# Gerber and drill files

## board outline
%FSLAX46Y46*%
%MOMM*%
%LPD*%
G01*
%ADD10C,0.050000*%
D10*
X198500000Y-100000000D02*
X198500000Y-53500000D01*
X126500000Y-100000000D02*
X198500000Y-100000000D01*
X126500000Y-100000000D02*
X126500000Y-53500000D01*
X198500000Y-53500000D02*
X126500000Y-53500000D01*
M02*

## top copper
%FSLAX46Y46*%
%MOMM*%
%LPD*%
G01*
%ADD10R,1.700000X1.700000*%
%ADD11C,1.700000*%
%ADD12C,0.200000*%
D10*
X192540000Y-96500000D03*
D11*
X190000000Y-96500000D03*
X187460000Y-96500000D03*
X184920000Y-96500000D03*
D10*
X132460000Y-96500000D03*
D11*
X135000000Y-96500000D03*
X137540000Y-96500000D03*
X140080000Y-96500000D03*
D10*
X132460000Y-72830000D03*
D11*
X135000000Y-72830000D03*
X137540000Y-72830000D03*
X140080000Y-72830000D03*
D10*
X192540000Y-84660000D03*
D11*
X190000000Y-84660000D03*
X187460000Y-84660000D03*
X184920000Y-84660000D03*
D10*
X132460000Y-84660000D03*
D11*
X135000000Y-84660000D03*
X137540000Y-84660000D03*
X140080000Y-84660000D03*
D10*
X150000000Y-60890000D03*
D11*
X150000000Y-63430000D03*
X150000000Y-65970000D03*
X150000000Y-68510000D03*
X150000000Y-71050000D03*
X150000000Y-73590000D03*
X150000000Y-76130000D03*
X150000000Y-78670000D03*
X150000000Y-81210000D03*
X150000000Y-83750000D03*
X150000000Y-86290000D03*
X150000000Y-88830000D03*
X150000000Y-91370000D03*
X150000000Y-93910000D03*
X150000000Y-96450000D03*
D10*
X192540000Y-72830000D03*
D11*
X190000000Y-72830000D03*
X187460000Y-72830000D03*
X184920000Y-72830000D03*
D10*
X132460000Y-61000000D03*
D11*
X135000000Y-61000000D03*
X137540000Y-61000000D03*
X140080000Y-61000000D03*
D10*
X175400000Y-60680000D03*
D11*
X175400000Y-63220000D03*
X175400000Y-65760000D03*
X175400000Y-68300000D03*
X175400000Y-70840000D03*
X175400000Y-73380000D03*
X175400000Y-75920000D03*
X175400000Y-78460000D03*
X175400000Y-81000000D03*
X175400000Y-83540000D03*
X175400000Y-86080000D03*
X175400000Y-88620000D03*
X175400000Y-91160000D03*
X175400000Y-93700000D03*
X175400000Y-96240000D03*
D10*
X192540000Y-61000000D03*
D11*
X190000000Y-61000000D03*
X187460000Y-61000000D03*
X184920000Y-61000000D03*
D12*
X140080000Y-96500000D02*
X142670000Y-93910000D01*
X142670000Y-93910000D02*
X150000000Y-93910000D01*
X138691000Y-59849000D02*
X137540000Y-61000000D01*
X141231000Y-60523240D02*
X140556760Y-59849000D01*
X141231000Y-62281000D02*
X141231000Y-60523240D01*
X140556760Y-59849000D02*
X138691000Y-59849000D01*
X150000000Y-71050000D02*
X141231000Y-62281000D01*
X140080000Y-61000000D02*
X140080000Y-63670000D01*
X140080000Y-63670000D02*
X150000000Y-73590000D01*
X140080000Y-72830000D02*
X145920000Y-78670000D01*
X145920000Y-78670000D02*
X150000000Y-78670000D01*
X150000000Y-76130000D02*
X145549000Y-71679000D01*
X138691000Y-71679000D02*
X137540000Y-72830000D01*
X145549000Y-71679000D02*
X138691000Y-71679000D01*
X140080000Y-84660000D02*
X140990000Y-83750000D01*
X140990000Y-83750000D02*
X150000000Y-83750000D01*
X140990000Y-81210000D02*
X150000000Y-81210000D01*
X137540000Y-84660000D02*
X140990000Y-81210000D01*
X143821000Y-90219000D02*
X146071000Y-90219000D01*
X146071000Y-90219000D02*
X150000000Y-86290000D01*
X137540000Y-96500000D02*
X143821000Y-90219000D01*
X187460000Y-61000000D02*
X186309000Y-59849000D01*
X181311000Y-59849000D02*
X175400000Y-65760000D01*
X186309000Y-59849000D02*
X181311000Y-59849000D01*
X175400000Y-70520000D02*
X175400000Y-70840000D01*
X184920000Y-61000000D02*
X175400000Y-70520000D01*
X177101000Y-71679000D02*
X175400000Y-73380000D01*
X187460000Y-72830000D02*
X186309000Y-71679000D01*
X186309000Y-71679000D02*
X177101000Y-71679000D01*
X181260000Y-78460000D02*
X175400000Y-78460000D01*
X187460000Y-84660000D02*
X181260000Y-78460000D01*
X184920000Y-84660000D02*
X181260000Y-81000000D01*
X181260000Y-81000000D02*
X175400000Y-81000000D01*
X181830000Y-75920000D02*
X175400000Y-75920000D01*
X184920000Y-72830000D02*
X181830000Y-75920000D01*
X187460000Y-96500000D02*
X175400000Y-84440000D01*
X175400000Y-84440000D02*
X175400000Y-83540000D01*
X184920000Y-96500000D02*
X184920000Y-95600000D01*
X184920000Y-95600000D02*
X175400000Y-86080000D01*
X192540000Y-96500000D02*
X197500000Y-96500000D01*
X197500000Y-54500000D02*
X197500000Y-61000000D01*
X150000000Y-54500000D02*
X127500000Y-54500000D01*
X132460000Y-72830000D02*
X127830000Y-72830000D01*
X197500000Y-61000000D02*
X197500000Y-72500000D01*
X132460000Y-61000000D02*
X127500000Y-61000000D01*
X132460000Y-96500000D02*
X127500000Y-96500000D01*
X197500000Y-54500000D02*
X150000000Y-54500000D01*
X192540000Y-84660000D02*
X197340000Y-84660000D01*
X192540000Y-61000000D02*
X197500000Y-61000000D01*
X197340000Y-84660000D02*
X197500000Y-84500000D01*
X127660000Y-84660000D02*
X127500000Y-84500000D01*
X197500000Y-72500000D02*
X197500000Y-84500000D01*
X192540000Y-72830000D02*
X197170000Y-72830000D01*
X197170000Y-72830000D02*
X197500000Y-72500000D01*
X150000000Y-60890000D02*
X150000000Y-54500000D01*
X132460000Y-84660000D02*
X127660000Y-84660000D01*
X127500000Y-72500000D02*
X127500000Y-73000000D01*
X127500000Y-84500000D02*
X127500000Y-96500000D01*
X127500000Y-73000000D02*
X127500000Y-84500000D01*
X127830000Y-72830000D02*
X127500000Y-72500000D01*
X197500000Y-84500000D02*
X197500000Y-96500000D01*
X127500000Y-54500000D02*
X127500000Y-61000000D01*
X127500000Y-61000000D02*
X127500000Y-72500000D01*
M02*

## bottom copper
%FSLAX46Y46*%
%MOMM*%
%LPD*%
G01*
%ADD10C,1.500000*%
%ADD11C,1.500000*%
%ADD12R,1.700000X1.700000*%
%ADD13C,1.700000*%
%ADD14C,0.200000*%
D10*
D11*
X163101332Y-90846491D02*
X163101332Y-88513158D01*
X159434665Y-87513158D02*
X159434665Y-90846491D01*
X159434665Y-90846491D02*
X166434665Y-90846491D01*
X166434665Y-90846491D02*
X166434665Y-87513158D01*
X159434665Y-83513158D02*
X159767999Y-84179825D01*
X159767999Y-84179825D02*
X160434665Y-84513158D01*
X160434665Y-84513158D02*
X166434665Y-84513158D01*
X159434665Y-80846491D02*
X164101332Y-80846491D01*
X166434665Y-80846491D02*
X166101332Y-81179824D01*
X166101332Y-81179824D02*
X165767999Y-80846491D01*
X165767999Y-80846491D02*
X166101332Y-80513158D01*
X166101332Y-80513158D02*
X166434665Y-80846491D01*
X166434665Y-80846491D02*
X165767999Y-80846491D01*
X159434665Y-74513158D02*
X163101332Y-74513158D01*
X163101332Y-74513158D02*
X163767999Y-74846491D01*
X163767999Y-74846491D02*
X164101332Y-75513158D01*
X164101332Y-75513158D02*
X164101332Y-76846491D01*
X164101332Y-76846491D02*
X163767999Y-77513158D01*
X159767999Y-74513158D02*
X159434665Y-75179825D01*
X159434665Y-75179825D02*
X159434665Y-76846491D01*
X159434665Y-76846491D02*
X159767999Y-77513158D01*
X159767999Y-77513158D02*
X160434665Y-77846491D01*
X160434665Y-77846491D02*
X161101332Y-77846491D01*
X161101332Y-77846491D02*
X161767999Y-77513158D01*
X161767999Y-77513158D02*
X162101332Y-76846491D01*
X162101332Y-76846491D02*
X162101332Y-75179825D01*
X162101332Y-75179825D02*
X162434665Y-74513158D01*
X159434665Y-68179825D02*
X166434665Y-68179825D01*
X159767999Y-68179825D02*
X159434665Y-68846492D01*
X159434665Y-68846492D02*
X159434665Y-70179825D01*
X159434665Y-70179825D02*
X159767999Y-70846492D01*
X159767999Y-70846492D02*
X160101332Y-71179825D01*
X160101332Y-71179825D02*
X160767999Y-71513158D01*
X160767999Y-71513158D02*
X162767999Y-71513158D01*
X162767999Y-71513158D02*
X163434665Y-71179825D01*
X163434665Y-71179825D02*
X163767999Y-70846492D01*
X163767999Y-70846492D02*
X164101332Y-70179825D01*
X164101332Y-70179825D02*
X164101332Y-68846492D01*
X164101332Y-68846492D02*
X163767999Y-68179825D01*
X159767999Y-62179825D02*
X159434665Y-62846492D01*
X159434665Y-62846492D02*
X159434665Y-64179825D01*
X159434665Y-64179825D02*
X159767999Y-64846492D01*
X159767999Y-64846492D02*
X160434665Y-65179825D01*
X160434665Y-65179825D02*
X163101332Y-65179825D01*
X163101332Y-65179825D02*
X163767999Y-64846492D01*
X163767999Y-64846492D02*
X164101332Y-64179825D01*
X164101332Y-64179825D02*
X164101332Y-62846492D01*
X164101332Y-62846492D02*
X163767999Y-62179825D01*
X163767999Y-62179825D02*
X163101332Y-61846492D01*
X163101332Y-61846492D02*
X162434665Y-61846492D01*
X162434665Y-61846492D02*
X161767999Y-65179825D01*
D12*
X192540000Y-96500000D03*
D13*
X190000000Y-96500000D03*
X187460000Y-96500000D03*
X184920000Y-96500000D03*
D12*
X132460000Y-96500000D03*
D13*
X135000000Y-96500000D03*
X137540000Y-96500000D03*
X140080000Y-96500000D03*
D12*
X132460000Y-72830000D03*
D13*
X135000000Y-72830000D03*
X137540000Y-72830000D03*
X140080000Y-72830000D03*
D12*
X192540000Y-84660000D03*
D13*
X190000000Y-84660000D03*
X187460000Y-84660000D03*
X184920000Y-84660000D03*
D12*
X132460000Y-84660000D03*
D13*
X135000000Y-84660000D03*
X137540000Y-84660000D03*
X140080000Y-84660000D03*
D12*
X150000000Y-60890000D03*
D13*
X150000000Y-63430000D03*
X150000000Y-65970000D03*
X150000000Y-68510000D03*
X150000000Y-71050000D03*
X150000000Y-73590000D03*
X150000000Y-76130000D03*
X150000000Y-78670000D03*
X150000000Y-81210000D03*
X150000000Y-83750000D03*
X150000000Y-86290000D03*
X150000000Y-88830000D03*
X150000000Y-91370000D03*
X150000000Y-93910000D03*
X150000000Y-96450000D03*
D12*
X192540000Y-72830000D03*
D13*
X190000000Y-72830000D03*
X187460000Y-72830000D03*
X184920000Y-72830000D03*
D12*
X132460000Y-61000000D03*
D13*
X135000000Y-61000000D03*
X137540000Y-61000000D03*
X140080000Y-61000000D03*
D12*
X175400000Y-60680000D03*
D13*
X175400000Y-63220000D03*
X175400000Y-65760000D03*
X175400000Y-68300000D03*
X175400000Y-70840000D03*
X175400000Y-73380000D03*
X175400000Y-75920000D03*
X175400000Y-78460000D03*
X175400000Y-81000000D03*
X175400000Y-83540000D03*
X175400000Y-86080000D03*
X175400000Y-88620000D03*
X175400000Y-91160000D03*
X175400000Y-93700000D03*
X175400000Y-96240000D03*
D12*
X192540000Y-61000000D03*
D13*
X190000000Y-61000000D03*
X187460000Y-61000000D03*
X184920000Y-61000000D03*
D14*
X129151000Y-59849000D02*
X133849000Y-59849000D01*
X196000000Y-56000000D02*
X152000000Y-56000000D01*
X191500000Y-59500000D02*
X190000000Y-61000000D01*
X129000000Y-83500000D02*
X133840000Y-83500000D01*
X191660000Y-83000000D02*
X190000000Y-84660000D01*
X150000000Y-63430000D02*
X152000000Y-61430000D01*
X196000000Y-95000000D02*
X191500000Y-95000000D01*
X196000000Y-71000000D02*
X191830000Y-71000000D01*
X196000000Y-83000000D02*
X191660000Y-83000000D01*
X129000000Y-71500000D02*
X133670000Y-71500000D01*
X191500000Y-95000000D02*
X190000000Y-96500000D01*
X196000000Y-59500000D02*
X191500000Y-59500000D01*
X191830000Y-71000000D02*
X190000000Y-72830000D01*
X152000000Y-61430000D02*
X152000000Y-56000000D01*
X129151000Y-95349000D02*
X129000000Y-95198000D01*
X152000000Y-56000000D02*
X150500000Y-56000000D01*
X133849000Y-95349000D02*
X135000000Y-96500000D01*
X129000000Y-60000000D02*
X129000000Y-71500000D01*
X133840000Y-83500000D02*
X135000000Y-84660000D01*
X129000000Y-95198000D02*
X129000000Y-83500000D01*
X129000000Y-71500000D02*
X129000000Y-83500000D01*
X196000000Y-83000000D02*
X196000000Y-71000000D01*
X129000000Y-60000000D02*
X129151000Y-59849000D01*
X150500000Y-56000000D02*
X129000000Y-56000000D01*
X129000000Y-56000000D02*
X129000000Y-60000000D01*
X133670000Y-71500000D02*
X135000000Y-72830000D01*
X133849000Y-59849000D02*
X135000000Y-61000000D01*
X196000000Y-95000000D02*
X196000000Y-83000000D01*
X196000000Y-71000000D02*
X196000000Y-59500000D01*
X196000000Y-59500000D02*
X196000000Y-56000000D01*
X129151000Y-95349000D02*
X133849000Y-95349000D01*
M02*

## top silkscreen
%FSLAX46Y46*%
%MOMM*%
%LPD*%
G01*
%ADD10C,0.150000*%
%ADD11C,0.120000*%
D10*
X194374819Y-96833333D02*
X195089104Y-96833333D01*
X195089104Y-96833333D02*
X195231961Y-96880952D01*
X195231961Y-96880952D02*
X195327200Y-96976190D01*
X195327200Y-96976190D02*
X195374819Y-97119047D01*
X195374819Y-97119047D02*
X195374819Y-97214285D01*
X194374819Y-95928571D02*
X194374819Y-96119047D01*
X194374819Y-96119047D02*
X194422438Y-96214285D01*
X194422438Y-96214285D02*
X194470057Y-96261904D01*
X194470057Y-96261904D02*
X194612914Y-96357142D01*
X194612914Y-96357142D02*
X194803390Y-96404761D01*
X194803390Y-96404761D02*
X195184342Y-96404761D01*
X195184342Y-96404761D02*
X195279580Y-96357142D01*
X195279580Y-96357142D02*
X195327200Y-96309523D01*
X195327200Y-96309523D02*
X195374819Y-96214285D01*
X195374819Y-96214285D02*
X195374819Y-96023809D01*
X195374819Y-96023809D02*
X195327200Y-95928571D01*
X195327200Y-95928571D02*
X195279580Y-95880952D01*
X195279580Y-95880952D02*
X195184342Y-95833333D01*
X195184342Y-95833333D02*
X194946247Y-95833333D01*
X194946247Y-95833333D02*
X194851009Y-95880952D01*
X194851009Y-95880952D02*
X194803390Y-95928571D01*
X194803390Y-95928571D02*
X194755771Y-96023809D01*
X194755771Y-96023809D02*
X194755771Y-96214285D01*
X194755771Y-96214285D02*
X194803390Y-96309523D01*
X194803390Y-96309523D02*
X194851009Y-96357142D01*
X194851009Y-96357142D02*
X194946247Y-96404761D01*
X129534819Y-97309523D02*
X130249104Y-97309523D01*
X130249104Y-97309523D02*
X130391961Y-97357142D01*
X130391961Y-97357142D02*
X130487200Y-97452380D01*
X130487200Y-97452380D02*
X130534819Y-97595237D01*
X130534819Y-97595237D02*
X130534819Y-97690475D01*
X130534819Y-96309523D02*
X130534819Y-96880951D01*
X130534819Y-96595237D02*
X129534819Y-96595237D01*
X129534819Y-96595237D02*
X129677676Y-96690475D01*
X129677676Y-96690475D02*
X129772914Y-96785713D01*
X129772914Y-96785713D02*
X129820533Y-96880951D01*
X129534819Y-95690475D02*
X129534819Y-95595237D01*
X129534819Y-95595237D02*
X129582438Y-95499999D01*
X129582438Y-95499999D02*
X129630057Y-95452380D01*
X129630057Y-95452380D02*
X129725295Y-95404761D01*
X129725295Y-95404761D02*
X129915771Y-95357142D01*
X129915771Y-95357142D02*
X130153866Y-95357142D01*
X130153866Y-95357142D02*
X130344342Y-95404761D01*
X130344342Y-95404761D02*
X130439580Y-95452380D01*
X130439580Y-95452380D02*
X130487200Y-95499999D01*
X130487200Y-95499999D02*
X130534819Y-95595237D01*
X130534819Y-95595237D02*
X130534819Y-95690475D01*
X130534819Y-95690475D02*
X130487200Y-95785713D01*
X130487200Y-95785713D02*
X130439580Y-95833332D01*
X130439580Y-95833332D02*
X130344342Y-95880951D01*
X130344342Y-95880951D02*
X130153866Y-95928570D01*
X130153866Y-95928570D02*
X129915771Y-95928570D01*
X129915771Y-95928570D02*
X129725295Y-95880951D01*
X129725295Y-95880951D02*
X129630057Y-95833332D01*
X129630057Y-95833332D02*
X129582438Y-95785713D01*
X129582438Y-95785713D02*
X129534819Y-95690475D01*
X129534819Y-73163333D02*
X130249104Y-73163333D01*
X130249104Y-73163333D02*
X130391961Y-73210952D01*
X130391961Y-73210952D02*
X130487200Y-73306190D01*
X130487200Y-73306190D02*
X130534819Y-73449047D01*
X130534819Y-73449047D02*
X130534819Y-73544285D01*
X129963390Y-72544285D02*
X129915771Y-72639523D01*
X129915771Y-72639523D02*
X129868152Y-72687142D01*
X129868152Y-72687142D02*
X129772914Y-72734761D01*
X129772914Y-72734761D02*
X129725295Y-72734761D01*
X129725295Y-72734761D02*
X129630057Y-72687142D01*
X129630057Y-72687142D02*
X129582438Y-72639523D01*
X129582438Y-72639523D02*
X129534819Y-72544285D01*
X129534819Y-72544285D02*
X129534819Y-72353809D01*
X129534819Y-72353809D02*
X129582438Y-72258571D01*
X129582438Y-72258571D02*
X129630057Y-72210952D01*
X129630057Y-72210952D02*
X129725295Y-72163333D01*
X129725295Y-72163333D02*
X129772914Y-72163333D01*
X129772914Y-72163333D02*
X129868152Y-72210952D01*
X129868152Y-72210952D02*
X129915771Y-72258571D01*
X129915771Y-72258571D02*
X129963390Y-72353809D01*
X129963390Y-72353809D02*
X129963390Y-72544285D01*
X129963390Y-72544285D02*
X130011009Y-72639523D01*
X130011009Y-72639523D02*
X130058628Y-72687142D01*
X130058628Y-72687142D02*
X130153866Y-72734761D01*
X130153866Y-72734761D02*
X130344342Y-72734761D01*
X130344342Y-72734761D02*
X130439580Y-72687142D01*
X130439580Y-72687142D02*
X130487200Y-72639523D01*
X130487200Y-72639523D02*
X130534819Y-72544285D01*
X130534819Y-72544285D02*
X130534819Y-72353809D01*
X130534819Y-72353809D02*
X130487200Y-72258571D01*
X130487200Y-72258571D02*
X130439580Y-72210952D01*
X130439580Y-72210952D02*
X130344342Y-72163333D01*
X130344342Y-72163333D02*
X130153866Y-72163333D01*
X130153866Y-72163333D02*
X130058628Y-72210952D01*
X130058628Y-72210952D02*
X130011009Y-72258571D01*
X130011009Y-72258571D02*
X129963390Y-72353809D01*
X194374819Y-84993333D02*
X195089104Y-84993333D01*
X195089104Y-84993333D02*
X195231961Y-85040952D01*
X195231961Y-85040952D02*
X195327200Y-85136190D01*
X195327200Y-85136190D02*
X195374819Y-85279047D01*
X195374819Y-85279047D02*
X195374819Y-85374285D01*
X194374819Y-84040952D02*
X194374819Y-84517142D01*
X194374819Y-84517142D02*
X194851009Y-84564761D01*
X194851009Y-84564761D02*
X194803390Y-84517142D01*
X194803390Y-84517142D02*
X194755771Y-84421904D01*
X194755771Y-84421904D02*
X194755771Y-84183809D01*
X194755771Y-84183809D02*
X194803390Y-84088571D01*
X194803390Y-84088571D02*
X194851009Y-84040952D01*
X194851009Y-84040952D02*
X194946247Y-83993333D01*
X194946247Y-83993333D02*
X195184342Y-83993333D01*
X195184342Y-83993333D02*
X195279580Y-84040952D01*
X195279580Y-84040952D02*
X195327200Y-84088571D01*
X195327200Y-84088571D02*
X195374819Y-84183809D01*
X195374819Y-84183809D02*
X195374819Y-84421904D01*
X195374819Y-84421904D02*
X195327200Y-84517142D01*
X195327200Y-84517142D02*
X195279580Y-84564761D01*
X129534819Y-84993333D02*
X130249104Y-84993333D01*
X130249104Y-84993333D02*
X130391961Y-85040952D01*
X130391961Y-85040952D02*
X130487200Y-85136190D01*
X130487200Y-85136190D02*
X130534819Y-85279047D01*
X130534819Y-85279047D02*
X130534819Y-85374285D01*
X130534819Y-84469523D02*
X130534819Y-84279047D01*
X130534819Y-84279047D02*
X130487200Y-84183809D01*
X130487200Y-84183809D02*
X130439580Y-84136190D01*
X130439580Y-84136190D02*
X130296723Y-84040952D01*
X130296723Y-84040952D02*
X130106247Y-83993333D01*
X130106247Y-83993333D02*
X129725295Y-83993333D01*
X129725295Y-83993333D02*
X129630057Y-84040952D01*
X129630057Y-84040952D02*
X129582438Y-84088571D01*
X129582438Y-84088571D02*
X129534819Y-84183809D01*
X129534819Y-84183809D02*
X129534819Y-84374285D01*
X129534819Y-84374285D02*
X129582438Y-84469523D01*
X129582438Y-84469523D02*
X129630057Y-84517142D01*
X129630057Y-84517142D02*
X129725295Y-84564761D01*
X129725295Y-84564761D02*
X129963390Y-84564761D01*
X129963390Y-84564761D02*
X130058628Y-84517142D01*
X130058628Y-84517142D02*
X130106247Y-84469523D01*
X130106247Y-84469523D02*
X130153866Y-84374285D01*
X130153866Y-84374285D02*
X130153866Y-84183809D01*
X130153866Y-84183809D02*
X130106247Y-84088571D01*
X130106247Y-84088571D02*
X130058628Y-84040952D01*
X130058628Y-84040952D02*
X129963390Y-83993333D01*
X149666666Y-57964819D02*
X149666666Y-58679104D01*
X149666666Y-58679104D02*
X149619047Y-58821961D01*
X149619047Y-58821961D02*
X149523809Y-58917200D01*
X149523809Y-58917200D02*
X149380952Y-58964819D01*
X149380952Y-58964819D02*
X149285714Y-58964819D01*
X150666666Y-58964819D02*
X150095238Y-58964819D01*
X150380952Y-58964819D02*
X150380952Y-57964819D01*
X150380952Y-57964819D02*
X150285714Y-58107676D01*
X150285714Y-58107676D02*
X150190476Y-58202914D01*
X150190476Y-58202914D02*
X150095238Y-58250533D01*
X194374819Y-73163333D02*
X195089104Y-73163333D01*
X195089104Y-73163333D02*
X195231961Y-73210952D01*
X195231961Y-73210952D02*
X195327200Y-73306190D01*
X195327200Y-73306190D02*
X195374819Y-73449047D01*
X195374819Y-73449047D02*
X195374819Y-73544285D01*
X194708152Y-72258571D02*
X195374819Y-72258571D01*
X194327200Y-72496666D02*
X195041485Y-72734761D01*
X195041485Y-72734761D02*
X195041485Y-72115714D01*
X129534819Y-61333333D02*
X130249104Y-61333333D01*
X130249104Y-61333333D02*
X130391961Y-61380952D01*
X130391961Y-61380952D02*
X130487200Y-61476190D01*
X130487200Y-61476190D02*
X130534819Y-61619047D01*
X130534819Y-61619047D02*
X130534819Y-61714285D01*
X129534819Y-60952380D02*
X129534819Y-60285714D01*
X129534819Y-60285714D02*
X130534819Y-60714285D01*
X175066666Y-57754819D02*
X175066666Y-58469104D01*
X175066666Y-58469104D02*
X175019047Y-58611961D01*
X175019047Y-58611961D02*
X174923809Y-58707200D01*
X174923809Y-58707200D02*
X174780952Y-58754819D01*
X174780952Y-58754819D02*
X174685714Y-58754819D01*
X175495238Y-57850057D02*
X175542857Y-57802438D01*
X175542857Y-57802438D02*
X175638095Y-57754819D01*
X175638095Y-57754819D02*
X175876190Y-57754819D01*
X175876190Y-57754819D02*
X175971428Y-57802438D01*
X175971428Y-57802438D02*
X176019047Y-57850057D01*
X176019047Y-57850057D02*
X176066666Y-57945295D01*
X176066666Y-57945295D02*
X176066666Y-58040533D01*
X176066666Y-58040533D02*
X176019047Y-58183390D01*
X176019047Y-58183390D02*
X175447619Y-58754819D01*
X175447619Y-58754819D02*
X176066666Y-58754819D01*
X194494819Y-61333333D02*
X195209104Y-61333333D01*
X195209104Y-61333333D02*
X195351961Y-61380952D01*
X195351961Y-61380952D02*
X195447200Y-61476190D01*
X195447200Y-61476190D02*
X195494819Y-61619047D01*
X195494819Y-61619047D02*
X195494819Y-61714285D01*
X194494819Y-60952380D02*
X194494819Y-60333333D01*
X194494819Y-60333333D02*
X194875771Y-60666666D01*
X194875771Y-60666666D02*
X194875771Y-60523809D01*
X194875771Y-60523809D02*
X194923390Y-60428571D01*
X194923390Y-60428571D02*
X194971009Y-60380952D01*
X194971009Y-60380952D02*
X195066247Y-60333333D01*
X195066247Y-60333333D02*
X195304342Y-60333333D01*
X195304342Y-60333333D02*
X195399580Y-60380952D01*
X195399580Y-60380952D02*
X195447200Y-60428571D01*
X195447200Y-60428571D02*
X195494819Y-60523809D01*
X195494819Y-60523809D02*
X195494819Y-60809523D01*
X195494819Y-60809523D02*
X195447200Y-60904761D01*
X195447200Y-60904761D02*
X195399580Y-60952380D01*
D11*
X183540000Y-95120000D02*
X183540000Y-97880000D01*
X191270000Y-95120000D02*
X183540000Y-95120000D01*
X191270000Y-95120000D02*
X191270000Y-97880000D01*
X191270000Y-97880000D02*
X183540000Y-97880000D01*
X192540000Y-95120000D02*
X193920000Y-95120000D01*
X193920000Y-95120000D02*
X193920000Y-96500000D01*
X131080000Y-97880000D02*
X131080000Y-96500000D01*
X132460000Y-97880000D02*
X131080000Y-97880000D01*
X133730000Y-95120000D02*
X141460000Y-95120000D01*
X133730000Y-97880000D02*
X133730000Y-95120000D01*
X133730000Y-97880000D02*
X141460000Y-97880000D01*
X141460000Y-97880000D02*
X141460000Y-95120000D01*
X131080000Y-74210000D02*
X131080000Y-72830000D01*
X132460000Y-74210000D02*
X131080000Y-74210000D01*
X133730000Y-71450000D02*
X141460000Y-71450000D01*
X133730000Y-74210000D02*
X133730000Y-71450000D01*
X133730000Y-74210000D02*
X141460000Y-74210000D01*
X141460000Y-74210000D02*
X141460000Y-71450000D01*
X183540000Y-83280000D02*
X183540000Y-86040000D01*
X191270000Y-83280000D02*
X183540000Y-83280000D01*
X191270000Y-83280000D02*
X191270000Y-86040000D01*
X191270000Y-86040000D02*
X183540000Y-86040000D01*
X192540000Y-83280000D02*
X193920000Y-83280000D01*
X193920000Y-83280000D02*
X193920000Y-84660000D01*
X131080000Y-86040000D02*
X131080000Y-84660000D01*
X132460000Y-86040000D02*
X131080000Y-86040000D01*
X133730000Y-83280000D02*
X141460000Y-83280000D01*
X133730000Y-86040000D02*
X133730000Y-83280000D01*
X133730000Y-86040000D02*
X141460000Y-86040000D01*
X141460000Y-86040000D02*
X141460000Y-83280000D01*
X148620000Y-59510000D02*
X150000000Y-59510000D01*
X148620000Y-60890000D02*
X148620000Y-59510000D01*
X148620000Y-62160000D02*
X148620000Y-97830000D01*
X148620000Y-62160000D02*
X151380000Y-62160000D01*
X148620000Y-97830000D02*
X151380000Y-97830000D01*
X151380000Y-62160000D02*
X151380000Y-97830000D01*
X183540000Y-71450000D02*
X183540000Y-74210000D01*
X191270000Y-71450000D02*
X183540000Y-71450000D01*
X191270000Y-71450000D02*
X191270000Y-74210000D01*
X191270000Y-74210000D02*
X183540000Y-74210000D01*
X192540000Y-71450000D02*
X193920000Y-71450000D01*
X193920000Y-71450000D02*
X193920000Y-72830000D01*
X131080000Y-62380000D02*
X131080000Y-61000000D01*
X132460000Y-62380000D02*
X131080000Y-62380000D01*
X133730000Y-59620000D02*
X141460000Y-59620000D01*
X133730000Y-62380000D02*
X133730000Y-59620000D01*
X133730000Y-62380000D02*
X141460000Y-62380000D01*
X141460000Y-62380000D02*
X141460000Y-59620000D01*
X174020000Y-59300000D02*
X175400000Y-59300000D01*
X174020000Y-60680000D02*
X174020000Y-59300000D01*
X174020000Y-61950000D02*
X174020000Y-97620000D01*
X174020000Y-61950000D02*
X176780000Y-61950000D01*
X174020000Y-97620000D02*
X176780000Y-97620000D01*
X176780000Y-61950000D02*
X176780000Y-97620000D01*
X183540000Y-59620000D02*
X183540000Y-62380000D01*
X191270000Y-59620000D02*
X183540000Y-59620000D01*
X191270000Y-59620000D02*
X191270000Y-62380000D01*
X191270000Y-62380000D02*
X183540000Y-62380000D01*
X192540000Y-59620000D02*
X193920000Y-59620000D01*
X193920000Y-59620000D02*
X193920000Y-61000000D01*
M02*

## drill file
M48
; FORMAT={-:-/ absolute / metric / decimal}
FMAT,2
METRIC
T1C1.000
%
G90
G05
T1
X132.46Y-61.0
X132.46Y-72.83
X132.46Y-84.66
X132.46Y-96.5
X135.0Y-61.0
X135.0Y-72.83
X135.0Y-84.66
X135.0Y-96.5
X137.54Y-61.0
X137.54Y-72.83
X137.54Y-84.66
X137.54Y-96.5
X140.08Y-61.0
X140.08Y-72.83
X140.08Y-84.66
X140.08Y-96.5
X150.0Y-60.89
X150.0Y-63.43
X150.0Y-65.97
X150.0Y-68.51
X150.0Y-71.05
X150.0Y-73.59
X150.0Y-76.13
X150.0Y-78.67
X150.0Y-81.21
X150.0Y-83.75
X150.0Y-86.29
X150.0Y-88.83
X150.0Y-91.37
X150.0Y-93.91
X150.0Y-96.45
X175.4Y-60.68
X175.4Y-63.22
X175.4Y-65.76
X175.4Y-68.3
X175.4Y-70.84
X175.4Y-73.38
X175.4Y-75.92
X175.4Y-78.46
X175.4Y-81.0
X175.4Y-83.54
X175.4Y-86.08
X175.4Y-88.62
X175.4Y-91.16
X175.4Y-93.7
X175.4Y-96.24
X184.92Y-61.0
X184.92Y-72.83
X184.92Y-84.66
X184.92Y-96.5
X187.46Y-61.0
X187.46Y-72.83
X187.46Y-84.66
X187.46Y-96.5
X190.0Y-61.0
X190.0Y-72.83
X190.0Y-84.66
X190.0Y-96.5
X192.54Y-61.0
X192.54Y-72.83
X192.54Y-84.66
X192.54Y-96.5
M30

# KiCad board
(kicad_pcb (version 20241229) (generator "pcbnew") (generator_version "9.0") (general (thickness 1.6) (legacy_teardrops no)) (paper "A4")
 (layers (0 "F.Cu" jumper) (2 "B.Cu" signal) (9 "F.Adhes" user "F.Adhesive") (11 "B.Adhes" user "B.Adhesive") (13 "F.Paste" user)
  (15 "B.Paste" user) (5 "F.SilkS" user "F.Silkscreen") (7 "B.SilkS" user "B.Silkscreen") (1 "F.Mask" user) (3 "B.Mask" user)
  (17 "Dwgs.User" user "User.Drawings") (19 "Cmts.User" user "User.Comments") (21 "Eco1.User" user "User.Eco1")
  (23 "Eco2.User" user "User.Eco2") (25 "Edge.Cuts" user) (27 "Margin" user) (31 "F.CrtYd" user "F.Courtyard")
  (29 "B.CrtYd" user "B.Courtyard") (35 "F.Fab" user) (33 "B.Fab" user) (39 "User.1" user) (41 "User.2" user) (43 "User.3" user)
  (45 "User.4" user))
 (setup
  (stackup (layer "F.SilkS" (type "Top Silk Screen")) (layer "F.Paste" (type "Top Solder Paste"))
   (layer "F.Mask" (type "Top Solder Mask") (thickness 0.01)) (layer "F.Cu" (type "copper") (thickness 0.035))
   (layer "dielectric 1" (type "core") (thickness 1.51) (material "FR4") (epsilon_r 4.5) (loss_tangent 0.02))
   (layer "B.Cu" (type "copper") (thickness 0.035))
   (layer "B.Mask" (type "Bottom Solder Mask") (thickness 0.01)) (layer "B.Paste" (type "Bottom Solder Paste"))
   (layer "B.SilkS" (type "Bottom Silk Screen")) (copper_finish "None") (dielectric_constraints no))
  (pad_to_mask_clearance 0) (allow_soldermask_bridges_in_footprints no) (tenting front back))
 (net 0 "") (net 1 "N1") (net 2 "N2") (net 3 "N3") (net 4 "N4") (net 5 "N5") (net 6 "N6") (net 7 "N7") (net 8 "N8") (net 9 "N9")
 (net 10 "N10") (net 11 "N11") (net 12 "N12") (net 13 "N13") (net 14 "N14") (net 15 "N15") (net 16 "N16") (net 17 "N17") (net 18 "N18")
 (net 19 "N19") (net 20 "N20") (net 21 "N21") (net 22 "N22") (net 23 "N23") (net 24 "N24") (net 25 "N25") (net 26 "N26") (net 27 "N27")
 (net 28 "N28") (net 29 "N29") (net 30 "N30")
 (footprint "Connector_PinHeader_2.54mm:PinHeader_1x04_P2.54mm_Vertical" (layer "F.Cu") (at 192.54 96.5 -90)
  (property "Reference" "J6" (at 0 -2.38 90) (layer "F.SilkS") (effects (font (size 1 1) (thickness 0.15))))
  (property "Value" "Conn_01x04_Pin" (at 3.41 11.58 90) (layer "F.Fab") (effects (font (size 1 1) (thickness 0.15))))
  (fp_line (start -1.38 9) (end 1.38 9) (stroke (width 0.12) (type solid)) (layer "F.SilkS"))
  (fp_line (start -1.38 1.27) (end -1.38 9) (stroke (width 0.12) (type solid)) (layer "F.SilkS"))
  (fp_line (start -1.38 1.27) (end 1.38 1.27) (stroke (width 0.12) (type solid)) (layer "F.SilkS"))
  (fp_line (start 1.38 1.27) (end 1.38 9) (stroke (width 0.12) (type solid)) (layer "F.SilkS"))
  (fp_line (start -1.38 0) (end -1.38 -1.38) (stroke (width 0.12) (type solid)) (layer "F.SilkS"))
  (fp_line (start -1.38 -1.38) (end 0 -1.38) (stroke (width 0.12) (type solid)) (layer "F.SilkS"))
  (pad "1" thru_hole rect (at 0 0 270) (size 1.7 1.7) (drill 1) (layers "*.Cu" "*.Mask") (remove_unused_layers no) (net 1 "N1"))
  (pad "2" thru_hole circle (at 0 2.54 270) (size 1.7 1.7) (drill 1) (layers "*.Cu" "*.Mask") (remove_unused_layers no) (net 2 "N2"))
  (pad "3" thru_hole circle (at 0 5.08 270) (size 1.7 1.7) (drill 1) (layers "*.Cu" "*.Mask") (remove_unused_layers no) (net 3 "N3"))
  (pad "4" thru_hole circle (at 0 7.62 270) (size 1.7 1.7) (drill 1) (layers "*.Cu" "*.Mask") (remove_unused_layers no) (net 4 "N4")))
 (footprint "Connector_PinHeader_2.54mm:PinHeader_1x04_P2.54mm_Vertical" (layer "F.Cu") (at 132.46 96.5 90)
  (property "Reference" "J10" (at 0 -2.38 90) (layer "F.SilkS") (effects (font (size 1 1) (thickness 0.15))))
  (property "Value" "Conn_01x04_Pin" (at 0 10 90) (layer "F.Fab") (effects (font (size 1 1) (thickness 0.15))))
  (fp_line (start -1.38 -1.38) (end 0 -1.38) (stroke (width 0.12) (type solid)) (layer "F.SilkS"))
  (fp_line (start -1.38 0) (end -1.38 -1.38) (stroke (width 0.12) (type solid)) (layer "F.SilkS"))
  (fp_line (start 1.38 1.27) (end 1.38 9) (stroke (width 0.12) (type solid)) (layer "F.SilkS"))
  (fp_line (start -1.38 1.27) (end 1.38 1.27) (stroke (width 0.12) (type solid)) (layer "F.SilkS"))
  (fp_line (start -1.38 1.27) (end -1.38 9) (stroke (width 0.12) (type solid)) (layer "F.SilkS"))
  (fp_line (start -1.38 9) (end 1.38 9) (stroke (width 0.12) (type solid)) (layer "F.SilkS"))
  (pad "1" thru_hole rect (at 0 0 90) (size 1.7 1.7) (drill 1) (layers "*.Cu" "*.Mask") (remove_unused_layers no) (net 1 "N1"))
  (pad "2" thru_hole circle (at 0 2.54 90) (size 1.7 1.7) (drill 1) (layers "*.Cu" "*.Mask") (remove_unused_layers no) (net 2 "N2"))
  (pad "3" thru_hole circle (at 0 5.08 90) (size 1.7 1.7) (drill 1) (layers "*.Cu" "*.Mask") (remove_unused_layers no) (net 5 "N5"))
  (pad "4" thru_hole circle (at 0 7.62 90) (size 1.7 1.7) (drill 1) (layers "*.Cu" "*.Mask") (remove_unused_layers no) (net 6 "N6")))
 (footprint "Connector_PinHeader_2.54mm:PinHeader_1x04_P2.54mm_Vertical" (layer "F.Cu") (at 132.46 72.83 90)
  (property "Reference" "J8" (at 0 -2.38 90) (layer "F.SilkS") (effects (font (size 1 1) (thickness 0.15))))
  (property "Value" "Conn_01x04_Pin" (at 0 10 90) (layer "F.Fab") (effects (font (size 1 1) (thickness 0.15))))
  (fp_line (start -1.38 -1.38) (end 0 -1.38) (stroke (width 0.12) (type solid)) (layer "F.SilkS"))
  (fp_line (start -1.38 0) (end -1.38 -1.38) (stroke (width 0.12) (type solid)) (layer "F.SilkS"))
  (fp_line (start 1.38 1.27) (end 1.38 9) (stroke (width 0.12) (type solid)) (layer "F.SilkS"))
  (fp_line (start -1.38 1.27) (end 1.38 1.27) (stroke (width 0.12) (type solid)) (layer "F.SilkS"))
  (fp_line (start -1.38 1.27) (end -1.38 9) (stroke (width 0.12) (type solid)) (layer "F.SilkS"))
  (fp_line (start -1.38 9) (end 1.38 9) (stroke (width 0.12) (type solid)) (layer "F.SilkS"))
  (pad "1" thru_hole rect (at 0 0 90) (size 1.7 1.7) (drill 1) (layers "*.Cu" "*.Mask") (remove_unused_layers no) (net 1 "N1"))
  (pad "2" thru_hole circle (at 0 2.54 90) (size 1.7 1.7) (drill 1) (layers "*.Cu" "*.Mask") (remove_unused_layers no) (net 2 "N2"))
  (pad "3" thru_hole circle (at 0 5.08 90) (size 1.7 1.7) (drill 1) (layers "*.Cu" "*.Mask") (remove_unused_layers no) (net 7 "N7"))
  (pad "4" thru_hole circle (at 0 7.62 90) (size 1.7 1.7) (drill 1) (layers "*.Cu" "*.Mask") (remove_unused_layers no) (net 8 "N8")))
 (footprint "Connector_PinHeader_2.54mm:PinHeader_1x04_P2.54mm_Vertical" (layer "F.Cu") (at 192.54 84.66 -90)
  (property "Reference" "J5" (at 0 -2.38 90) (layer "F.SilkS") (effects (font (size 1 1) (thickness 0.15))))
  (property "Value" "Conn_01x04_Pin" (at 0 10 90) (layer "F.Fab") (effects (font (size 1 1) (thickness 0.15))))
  (fp_line (start -1.38 9) (end 1.38 9) (stroke (width 0.12) (type solid)) (layer "F.SilkS"))
  (fp_line (start -1.38 1.27) (end -1.38 9) (stroke (width 0.12) (type solid)) (layer "F.SilkS"))
  (fp_line (start -1.38 1.27) (end 1.38 1.27) (stroke (width 0.12) (type solid)) (layer "F.SilkS"))
  (fp_line (start 1.38 1.27) (end 1.38 9) (stroke (width 0.12) (type solid)) (layer "F.SilkS"))
  (fp_line (start -1.38 0) (end -1.38 -1.38) (stroke (width 0.12) (type solid)) (layer "F.SilkS"))
  (fp_line (start -1.38 -1.38) (end 0 -1.38) (stroke (width 0.12) (type solid)) (layer "F.SilkS"))
  (pad "1" thru_hole rect (at 0 0 270) (size 1.7 1.7) (drill 1) (layers "*.Cu" "*.Mask") (remove_unused_layers no) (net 1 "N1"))
  (pad "2" thru_hole circle (at 0 2.54 270) (size 1.7 1.7) (drill 1) (layers "*.Cu" "*.Mask") (remove_unused_layers no) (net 2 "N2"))
  (pad "3" thru_hole circle (at 0 5.08 270) (size 1.7 1.7) (drill 1) (layers "*.Cu" "*.Mask") (remove_unused_layers no) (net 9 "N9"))
  (pad "4" thru_hole circle (at 0 7.62 270) (size 1.7 1.7) (drill 1) (layers "*.Cu" "*.Mask") (remove_unused_layers no) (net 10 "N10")))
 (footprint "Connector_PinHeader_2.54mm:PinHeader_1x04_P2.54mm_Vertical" (layer "F.Cu") (at 132.46 84.66 90)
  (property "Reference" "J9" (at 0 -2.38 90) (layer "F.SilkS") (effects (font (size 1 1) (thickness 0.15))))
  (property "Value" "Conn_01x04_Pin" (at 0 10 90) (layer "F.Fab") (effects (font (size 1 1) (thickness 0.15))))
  (fp_line (start -1.38 -1.38) (end 0 -1.38) (stroke (width 0.12) (type solid)) (layer "F.SilkS"))
  (fp_line (start -1.38 0) (end -1.38 -1.38) (stroke (width 0.12) (type solid)) (layer "F.SilkS"))
  (fp_line (start 1.38 1.27) (end 1.38 9) (stroke (width 0.12) (type solid)) (layer "F.SilkS"))
  (fp_line (start -1.38 1.27) (end 1.38 1.27) (stroke (width 0.12) (type solid)) (layer "F.SilkS"))
  (fp_line (start -1.38 1.27) (end -1.38 9) (stroke (width 0.12) (type solid)) (layer "F.SilkS"))
  (fp_line (start -1.38 9) (end 1.38 9) (stroke (width 0.12) (type solid)) (layer "F.SilkS"))
  (pad "1" thru_hole rect (at 0 0 90) (size 1.7 1.7) (drill 1) (layers "*.Cu" "*.Mask") (remove_unused_layers no) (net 1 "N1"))
  (pad "2" thru_hole circle (at 0 2.54 90) (size 1.7 1.7) (drill 1) (layers "*.Cu" "*.Mask") (remove_unused_layers no) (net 2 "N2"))
  (pad "3" thru_hole circle (at 0 5.08 90) (size 1.7 1.7) (drill 1) (layers "*.Cu" "*.Mask") (remove_unused_layers no) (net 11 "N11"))
  (pad "4" thru_hole circle (at 0 7.62 90) (size 1.7 1.7) (drill 1) (layers "*.Cu" "*.Mask") (remove_unused_layers no) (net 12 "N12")))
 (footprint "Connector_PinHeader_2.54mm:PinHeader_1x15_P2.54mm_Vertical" (layer "F.Cu") (at 150 60.89)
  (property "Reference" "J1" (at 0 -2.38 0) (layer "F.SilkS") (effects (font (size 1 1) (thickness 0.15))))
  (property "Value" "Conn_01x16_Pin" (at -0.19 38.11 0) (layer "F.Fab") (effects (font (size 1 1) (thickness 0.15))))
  (fp_line (start -1.38 -1.38) (end 0 -1.38) (stroke (width 0.12) (type solid)) (layer "F.SilkS"))
  (fp_line (start -1.38 0) (end -1.38 -1.38) (stroke (width 0.12) (type solid)) (layer "F.SilkS"))
  (fp_line (start -1.38 1.27) (end -1.38 36.94) (stroke (width 0.12) (type solid)) (layer "F.SilkS"))
  (fp_line (start -1.38 1.27) (end 1.38 1.27) (stroke (width 0.12) (type solid)) (layer "F.SilkS"))
  (fp_line (start -1.38 36.94) (end 1.38 36.94) (stroke (width 0.12) (type solid)) (layer "F.SilkS"))
  (fp_line (start 1.38 1.27) (end 1.38 36.94) (stroke (width 0.12) (type solid)) (layer "F.SilkS"))
  (pad "1" thru_hole rect (at 0 0) (size 1.7 1.7) (drill 1) (layers "*.Cu" "*.Mask") (remove_unused_layers no) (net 1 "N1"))
  (pad "2" thru_hole circle (at 0 2.54) (size 1.7 1.7) (drill 1) (layers "*.Cu" "*.Mask") (remove_unused_layers no) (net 2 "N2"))
  (pad "3" thru_hole circle (at 0 5.08) (size 1.7 1.7) (drill 1) (layers "*.Cu" "*.Mask") (remove_unused_layers no) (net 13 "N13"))
  (pad "4" thru_hole circle (at 0 7.62) (size 1.7 1.7) (drill 1) (layers "*.Cu" "*.Mask") (remove_unused_layers no) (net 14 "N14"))
  (pad "5" thru_hole circle (at 0 10.16) (size 1.7 1.7) (drill 1) (layers "*.Cu" "*.Mask") (remove_unused_layers no) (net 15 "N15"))
  (pad "6" thru_hole circle (at 0 12.7) (size 1.7 1.7) (drill 1) (layers "*.Cu" "*.Mask") (remove_unused_layers no) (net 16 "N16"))
  (pad "7" thru_hole circle (at 0 15.24) (size 1.7 1.7) (drill 1) (layers "*.Cu" "*.Mask") (remove_unused_layers no) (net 7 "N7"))
  (pad "8" thru_hole circle (at 0 17.78) (size 1.7 1.7) (drill 1) (layers "*.Cu" "*.Mask") (remove_unused_layers no) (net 8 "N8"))
  (pad "9" thru_hole circle (at 0 20.32) (size 1.7 1.7) (drill 1) (layers "*.Cu" "*.Mask") (remove_unused_layers no) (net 11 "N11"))
  (pad "10" thru_hole circle (at 0 22.86) (size 1.7 1.7) (drill 1) (layers "*.Cu" "*.Mask") (remove_unused_layers no) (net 12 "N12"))
  (pad "11" thru_hole circle (at 0 25.4) (size 1.7 1.7) (drill 1) (layers "*.Cu" "*.Mask") (remove_unused_layers no) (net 5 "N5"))
  (pad "12" thru_hole circle (at 0 27.94) (size 1.7 1.7) (drill 1) (layers "*.Cu" "*.Mask") (remove_unused_layers no) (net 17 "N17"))
  (pad "13" thru_hole circle (at 0 30.48) (size 1.7 1.7) (drill 1) (layers "*.Cu" "*.Mask") (remove_unused_layers no) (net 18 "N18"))
  (pad "14" thru_hole circle (at 0 33.02) (size 1.7 1.7) (drill 1) (layers "*.Cu" "*.Mask") (remove_unused_layers no) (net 6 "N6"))
  (pad "15" thru_hole circle (at 0 35.56) (size 1.7 1.7) (drill 1) (layers "*.Cu" "*.Mask") (remove_unused_layers no) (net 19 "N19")))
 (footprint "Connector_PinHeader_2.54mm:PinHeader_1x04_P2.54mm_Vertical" (layer "F.Cu") (at 192.54 72.83 -90)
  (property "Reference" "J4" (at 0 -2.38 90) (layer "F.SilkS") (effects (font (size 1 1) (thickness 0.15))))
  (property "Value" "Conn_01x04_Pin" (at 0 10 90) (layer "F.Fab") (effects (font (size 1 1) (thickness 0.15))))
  (fp_line (start -1.38 9) (end 1.38 9) (stroke (width 0.12) (type solid)) (layer "F.SilkS"))
  (fp_line (start -1.38 1.27) (end -1.38 9) (stroke (width 0.12) (type solid)) (layer "F.SilkS"))
  (fp_line (start -1.38 1.27) (end 1.38 1.27) (stroke (width 0.12) (type solid)) (layer "F.SilkS"))
  (fp_line (start 1.38 1.27) (end 1.38 9) (stroke (width 0.12) (type solid)) (layer "F.SilkS"))
  (fp_line (start -1.38 0) (end -1.38 -1.38) (stroke (width 0.12) (type solid)) (layer "F.SilkS"))
  (fp_line (start -1.38 -1.38) (end 0 -1.38) (stroke (width 0.12) (type solid)) (layer "F.SilkS"))
  (pad "1" thru_hole rect (at 0 0 270) (size 1.7 1.7) (drill 1) (layers "*.Cu" "*.Mask") (remove_unused_layers no) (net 1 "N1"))
  (pad "2" thru_hole circle (at 0 2.54 270) (size 1.7 1.7) (drill 1) (layers "*.Cu" "*.Mask") (remove_unused_layers no) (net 2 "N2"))
  (pad "3" thru_hole circle (at 0 5.08 270) (size 1.7 1.7) (drill 1) (layers "*.Cu" "*.Mask") (remove_unused_layers no) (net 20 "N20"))
  (pad "4" thru_hole circle (at 0 7.62 270) (size 1.7 1.7) (drill 1) (layers "*.Cu" "*.Mask") (remove_unused_layers no) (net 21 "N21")))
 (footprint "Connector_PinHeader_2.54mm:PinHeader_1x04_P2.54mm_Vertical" (layer "F.Cu") (at 132.46 61 90)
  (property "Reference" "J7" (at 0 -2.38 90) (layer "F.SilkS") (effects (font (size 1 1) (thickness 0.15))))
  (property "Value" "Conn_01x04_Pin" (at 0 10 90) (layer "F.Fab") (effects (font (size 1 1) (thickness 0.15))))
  (fp_line (start -1.38 -1.38) (end 0 -1.38) (stroke (width 0.12) (type solid)) (layer "F.SilkS"))
  (fp_line (start -1.38 0) (end -1.38 -1.38) (stroke (width 0.12) (type solid)) (layer "F.SilkS"))
  (fp_line (start 1.38 1.27) (end 1.38 9) (stroke (width 0.12) (type solid)) (layer "F.SilkS"))
  (fp_line (start -1.38 1.27) (end 1.38 1.27) (stroke (width 0.12) (type solid)) (layer "F.SilkS"))
  (fp_line (start -1.38 1.27) (end -1.38 9) (stroke (width 0.12) (type solid)) (layer "F.SilkS"))
  (fp_line (start -1.38 9) (end 1.38 9) (stroke (width 0.12) (type solid)) (layer "F.SilkS"))
  (pad "1" thru_hole rect (at 0 0 90) (size 1.7 1.7) (drill 1) (layers "*.Cu" "*.Mask") (remove_unused_layers no) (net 1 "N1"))
  (pad "2" thru_hole circle (at 0 2.54 90) (size 1.7 1.7) (drill 1) (layers "*.Cu" "*.Mask") (remove_unused_layers no) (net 2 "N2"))
  (pad "3" thru_hole circle (at 0 5.08 90) (size 1.7 1.7) (drill 1) (layers "*.Cu" "*.Mask") (remove_unused_layers no) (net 15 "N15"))
  (pad "4" thru_hole circle (at 0 7.62 90) (size 1.7 1.7) (drill 1) (layers "*.Cu" "*.Mask") (remove_unused_layers no) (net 16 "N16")))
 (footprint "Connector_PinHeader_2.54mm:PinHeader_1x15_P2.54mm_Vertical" (layer "F.Cu") (at 175.4 60.68)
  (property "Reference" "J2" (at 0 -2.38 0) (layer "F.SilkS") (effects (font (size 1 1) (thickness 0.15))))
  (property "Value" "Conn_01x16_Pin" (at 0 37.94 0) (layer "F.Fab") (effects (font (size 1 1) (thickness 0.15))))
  (fp_line (start -1.38 -1.38) (end 0 -1.38) (stroke (width 0.12) (type solid)) (layer "F.SilkS"))
  (fp_line (start -1.38 0) (end -1.38 -1.38) (stroke (width 0.12) (type solid)) (layer "F.SilkS"))
  (fp_line (start -1.38 1.27) (end -1.38 36.94) (stroke (width 0.12) (type solid)) (layer "F.SilkS"))
  (fp_line (start -1.38 1.27) (end 1.38 1.27) (stroke (width 0.12) (type solid)) (layer "F.SilkS"))
  (fp_line (start -1.38 36.94) (end 1.38 36.94) (stroke (width 0.12) (type solid)) (layer "F.SilkS"))
  (fp_line (start 1.38 1.27) (end 1.38 36.94) (stroke (width 0.12) (type solid)) (layer "F.SilkS"))
  (pad "1" thru_hole rect (at 0 0) (size 1.7 1.7) (drill 1) (layers "*.Cu" "*.Mask") (remove_unused_layers no) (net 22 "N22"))
  (pad "2" thru_hole circle (at 0 2.54) (size 1.7 1.7) (drill 1) (layers "*.Cu" "*.Mask") (remove_unused_layers no) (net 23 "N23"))
  (pad "3" thru_hole circle (at 0 5.08) (size 1.7 1.7) (drill 1) (layers "*.Cu" "*.Mask") (remove_unused_layers no) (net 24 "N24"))
  (pad "4" thru_hole circle (at 0 7.62) (size 1.7 1.7) (drill 1) (layers "*.Cu" "*.Mask") (remove_unused_layers no) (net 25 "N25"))
  (pad "5" thru_hole circle (at 0 10.16) (size 1.7 1.7) (drill 1) (layers "*.Cu" "*.Mask") (remove_unused_layers no) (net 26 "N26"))
  (pad "6" thru_hole circle (at 0 12.7) (size 1.7 1.7) (drill 1) (layers "*.Cu" "*.Mask") (remove_unused_layers no) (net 20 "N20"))
  (pad "7" thru_hole circle (at 0 15.24) (size 1.7 1.7) (drill 1) (layers "*.Cu" "*.Mask") (remove_unused_layers no) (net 21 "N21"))
  (pad "8" thru_hole circle (at 0 17.78) (size 1.7 1.7) (drill 1) (layers "*.Cu" "*.Mask") (remove_unused_layers no) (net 9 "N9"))
  (pad "9" thru_hole circle (at 0 20.32) (size 1.7 1.7) (drill 1) (layers "*.Cu" "*.Mask") (remove_unused_layers no) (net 10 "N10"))
  (pad "10" thru_hole circle (at 0 22.86) (size 1.7 1.7) (drill 1) (layers "*.Cu" "*.Mask") (remove_unused_layers no) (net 3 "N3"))
  (pad "11" thru_hole circle (at 0 25.4) (size 1.7 1.7) (drill 1) (layers "*.Cu" "*.Mask") (remove_unused_layers no) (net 4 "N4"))
  (pad "12" thru_hole circle (at 0 27.94) (size 1.7 1.7) (drill 1) (layers "*.Cu" "*.Mask") (remove_unused_layers no) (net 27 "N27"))
  (pad "13" thru_hole circle (at 0 30.48) (size 1.7 1.7) (drill 1) (layers "*.Cu" "*.Mask") (remove_unused_layers no) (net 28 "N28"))
  (pad "14" thru_hole circle (at 0 33.02) (size 1.7 1.7) (drill 1) (layers "*.Cu" "*.Mask") (remove_unused_layers no) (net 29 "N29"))
  (pad "15" thru_hole circle (at 0 35.56) (size 1.7 1.7) (drill 1) (layers "*.Cu" "*.Mask") (remove_unused_layers no) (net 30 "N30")))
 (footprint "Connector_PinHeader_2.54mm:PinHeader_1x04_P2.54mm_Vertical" (layer "F.Cu") (at 192.54 61 -90)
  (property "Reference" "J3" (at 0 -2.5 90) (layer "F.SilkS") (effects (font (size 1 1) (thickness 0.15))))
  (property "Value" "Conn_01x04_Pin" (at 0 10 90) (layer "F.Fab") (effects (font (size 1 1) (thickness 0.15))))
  (fp_line (start -1.38 9) (end 1.38 9) (stroke (width 0.12) (type solid)) (layer "F.SilkS"))
  (fp_line (start -1.38 1.27) (end -1.38 9) (stroke (width 0.12) (type solid)) (layer "F.SilkS"))
  (fp_line (start -1.38 1.27) (end 1.38 1.27) (stroke (width 0.12) (type solid)) (layer "F.SilkS"))
  (fp_line (start 1.38 1.27) (end 1.38 9) (stroke (width 0.12) (type solid)) (layer "F.SilkS"))
  (fp_line (start -1.38 0) (end -1.38 -1.38) (stroke (width 0.12) (type solid)) (layer "F.SilkS"))
  (fp_line (start -1.38 -1.38) (end 0 -1.38) (stroke (width 0.12) (type solid)) (layer "F.SilkS"))
  (pad "1" thru_hole rect (at 0 0 270) (size 1.7 1.7) (drill 1) (layers "*.Cu" "*.Mask") (remove_unused_layers no) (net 1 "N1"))
  (pad "2" thru_hole circle (at 0 2.54 270) (size 1.7 1.7) (drill 1) (layers "*.Cu" "*.Mask") (remove_unused_layers no) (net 2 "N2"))
  (pad "3" thru_hole circle (at 0 5.08 270) (size 1.7 1.7) (drill 1) (layers "*.Cu" "*.Mask") (remove_unused_layers no) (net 24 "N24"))
  (pad "4" thru_hole circle (at 0 7.62 270) (size 1.7 1.7) (drill 1) (layers "*.Cu" "*.Mask") (remove_unused_layers no) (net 26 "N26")))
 (gr_line (start 198.5 100) (end 198.5 53.5) (stroke (width 0.05) (type default)) (layer "Edge.Cuts"))
 (gr_line (start 126.5 100) (end 198.5 100) (stroke (width 0.05) (type default)) (layer "Edge.Cuts"))
 (gr_line (start 126.5 100) (end 126.5 53.5) (stroke (width 0.05) (type default)) (layer "Edge.Cuts"))
 (gr_line (start 198.5 53.5) (end 126.5 53.5) (stroke (width 0.05) (type default)) (layer "Edge.Cuts"))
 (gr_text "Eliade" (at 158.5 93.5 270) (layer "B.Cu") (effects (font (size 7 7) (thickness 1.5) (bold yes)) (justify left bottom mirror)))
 (segment (start 140.08 96.5) (end 142.67 93.91) (width 0.2) (layer "F.Cu") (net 6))
 (segment (start 142.67 93.91) (end 150 93.91) (width 0.2) (layer "F.Cu") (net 6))
 (segment (start 138.691 59.849) (end 137.54 61) (width 0.2) (layer "F.Cu") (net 15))
 (segment (start 141.231 60.52324) (end 140.55676 59.849) (width 0.2) (layer "F.Cu") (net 15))
 (segment (start 141.231 62.281) (end 141.231 60.52324) (width 0.2) (layer "F.Cu") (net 15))
 (segment (start 140.55676 59.849) (end 138.691 59.849) (width 0.2) (layer "F.Cu") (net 15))
 (segment (start 150 71.05) (end 141.231 62.281) (width 0.2) (layer "F.Cu") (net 15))
 (segment (start 140.08 61) (end 140.08 63.67) (width 0.2) (layer "F.Cu") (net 16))
 (segment (start 140.08 63.67) (end 150 73.59) (width 0.2) (layer "F.Cu") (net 16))
 (segment (start 140.08 72.83) (end 145.92 78.67) (width 0.2) (layer "F.Cu") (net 8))
 (segment (start 145.92 78.67) (end 150 78.67) (width 0.2) (layer "F.Cu") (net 8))
 (segment (start 150 76.13) (end 145.549 71.679) (width 0.2) (layer "F.Cu") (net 7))
 (segment (start 138.691 71.679) (end 137.54 72.83) (width 0.2) (layer "F.Cu") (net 7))
 (segment (start 145.549 71.679) (end 138.691 71.679) (width 0.2) (layer "F.Cu") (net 7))
 (segment (start 140.08 84.66) (end 140.99 83.75) (width 0.2) (layer "F.Cu") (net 12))
 (segment (start 140.99 83.75) (end 150 83.75) (width 0.2) (layer "F.Cu") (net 12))
 (segment (start 140.99 81.21) (end 150 81.21) (width 0.2) (layer "F.Cu") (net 11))
 (segment (start 137.54 84.66) (end 140.99 81.21) (width 0.2) (layer "F.Cu") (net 11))
 (segment (start 143.821 90.219) (end 146.071 90.219) (width 0.2) (layer "F.Cu") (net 5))
 (segment (start 146.071 90.219) (end 150 86.29) (width 0.2) (layer "F.Cu") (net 5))
 (segment (start 137.54 96.5) (end 143.821 90.219) (width 0.2) (layer "F.Cu") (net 5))
 (segment (start 187.46 61) (end 186.309 59.849) (width 0.2) (layer "F.Cu") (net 24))
 (segment (start 181.311 59.849) (end 175.4 65.76) (width 0.2) (layer "F.Cu") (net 24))
 (segment (start 186.309 59.849) (end 181.311 59.849) (width 0.2) (layer "F.Cu") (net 24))
 (segment (start 175.4 70.52) (end 175.4 70.84) (width 0.2) (layer "F.Cu") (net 26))
 (segment (start 184.92 61) (end 175.4 70.52) (width 0.2) (layer "F.Cu") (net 26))
 (segment (start 177.101 71.679) (end 175.4 73.38) (width 0.2) (layer "F.Cu") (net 20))
 (segment (start 187.46 72.83) (end 186.309 71.679) (width 0.2) (layer "F.Cu") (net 20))
 (segment (start 186.309 71.679) (end 177.101 71.679) (width 0.2) (layer "F.Cu") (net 20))
 (segment (start 181.26 78.46) (end 175.4 78.46) (width 0.2) (layer "F.Cu") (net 9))
 (segment (start 187.46 84.66) (end 181.26 78.46) (width 0.2) (layer "F.Cu") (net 9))
 (segment (start 184.92 84.66) (end 181.26 81) (width 0.2) (layer "F.Cu") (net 10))
 (segment (start 181.26 81) (end 175.4 81) (width 0.2) (layer "F.Cu") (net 10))
 (segment (start 181.83 75.92) (end 175.4 75.92) (width 0.2) (layer "F.Cu") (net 21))
 (segment (start 184.92 72.83) (end 181.83 75.92) (width 0.2) (layer "F.Cu") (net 21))
 (segment (start 187.46 96.5) (end 175.4 84.44) (width 0.2) (layer "F.Cu") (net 3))
 (segment (start 175.4 84.44) (end 175.4 83.54) (width 0.2) (layer "F.Cu") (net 3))
 (segment (start 184.92 96.5) (end 184.92 95.6) (width 0.2) (layer "F.Cu") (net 4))
 (segment (start 184.92 95.6) (end 175.4 86.08) (width 0.2) (layer "F.Cu") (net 4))
 (segment (start 129.151 59.849) (end 133.849 59.849) (width 0.2) (layer "B.Cu") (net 2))
 (segment (start 196 56) (end 152 56) (width 0.2) (layer "B.Cu") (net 2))
 (segment (start 191.5 59.5) (end 190 61) (width 0.2) (layer "B.Cu") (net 2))
 (segment (start 129 83.5) (end 133.84 83.5) (width 0.2) (layer "B.Cu") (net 2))
 (segment (start 191.66 83) (end 190 84.66) (width 0.2) (layer "B.Cu") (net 2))
 (segment (start 150 63.43) (end 152 61.43) (width 0.2) (layer "B.Cu") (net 2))
 (segment (start 196 95) (end 191.5 95) (width 0.2) (layer "B.Cu") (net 2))
 (segment (start 196 71) (end 191.83 71) (width 0.2) (layer "B.Cu") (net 2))
 (segment (start 196 83) (end 191.66 83) (width 0.2) (layer "B.Cu") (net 2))
 (segment (start 129 71.5) (end 133.67 71.5) (width 0.2) (layer "B.Cu") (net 2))
 (segment (start 191.5 95) (end 190 96.5) (width 0.2) (layer "B.Cu") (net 2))
 (segment (start 196 59.5) (end 191.5 59.5) (width 0.2) (layer "B.Cu") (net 2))
 (segment (start 191.83 71) (end 190 72.83) (width 0.2) (layer "B.Cu") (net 2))
 (segment (start 152 61.43) (end 152 56) (width 0.2) (layer "B.Cu") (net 2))
 (segment (start 129.151 95.349) (end 129 95.198) (width 0.2) (layer "B.Cu") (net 2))
 (segment (start 152 56) (end 150.5 56) (width 0.2) (layer "B.Cu") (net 2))
 (segment (start 133.849 95.349) (end 135 96.5) (width 0.2) (layer "B.Cu") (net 2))
 (segment (start 129 60) (end 129 71.5) (width 0.2) (layer "B.Cu") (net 2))
 (segment (start 133.84 83.5) (end 135 84.66) (width 0.2) (layer "B.Cu") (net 2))
 (segment (start 129 95.198) (end 129 83.5) (width 0.2) (layer "B.Cu") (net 2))
 (segment (start 129 71.5) (end 129 83.5) (width 0.2) (layer "B.Cu") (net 2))
 (segment (start 196 83) (end 196 71) (width 0.2) (layer "B.Cu") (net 2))
 (segment (start 129 60) (end 129.151 59.849) (width 0.2) (layer "B.Cu") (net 2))
 (segment (start 150.5 56) (end 129 56) (width 0.2) (layer "B.Cu") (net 2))
 (segment (start 129 56) (end 129 60) (width 0.2) (layer "B.Cu") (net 2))
 (segment (start 133.67 71.5) (end 135 72.83) (width 0.2) (layer "B.Cu") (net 2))
 (segment (start 133.849 59.849) (end 135 61) (width 0.2) (layer "B.Cu") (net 2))
 (segment (start 196 95) (end 196 83) (width 0.2) (layer "B.Cu") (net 2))
 (segment (start 196 71) (end 196 59.5) (width 0.2) (layer "B.Cu") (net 2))
 (segment (start 196 59.5) (end 196 56) (width 0.2) (layer "B.Cu") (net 2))
 (segment (start 129.151 95.349) (end 133.849 95.349) (width 0.2) (layer "B.Cu") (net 2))
 (segment (start 192.54 96.5) (end 197.5 96.5) (width 0.2) (layer "F.Cu") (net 1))
 (segment (start 197.5 54.5) (end 197.5 61) (width 0.2) (layer "F.Cu") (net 1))
 (segment (start 150 54.5) (end 127.5 54.5) (width 0.2) (layer "F.Cu") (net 1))
 (segment (start 132.46 72.83) (end 127.83 72.83) (width 0.2) (layer "F.Cu") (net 1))
 (segment (start 197.5 61) (end 197.5 72.5) (width 0.2) (layer "F.Cu") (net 1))
 (segment (start 132.46 61) (end 127.5 61) (width 0.2) (layer "F.Cu") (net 1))
 (segment (start 132.46 96.5) (end 127.5 96.5) (width 0.2) (layer "F.Cu") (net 1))
 (segment (start 197.5 54.5) (end 150 54.5) (width 0.2) (layer "F.Cu") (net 1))
 (segment (start 192.54 84.66) (end 197.34 84.66) (width 0.2) (layer "F.Cu") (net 1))
 (segment (start 192.54 61) (end 197.5 61) (width 0.2) (layer "F.Cu") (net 1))
 (segment (start 197.34 84.66) (end 197.5 84.5) (width 0.2) (layer "F.Cu") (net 1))
 (segment (start 127.66 84.66) (end 127.5 84.5) (width 0.2) (layer "F.Cu") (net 1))
 (segment (start 197.5 72.5) (end 197.5 84.5) (width 0.2) (layer "F.Cu") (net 1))
 (segment (start 192.54 72.83) (end 197.17 72.83) (width 0.2) (layer "F.Cu") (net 1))
 (segment (start 197.17 72.83) (end 197.5 72.5) (width 0.2) (layer "F.Cu") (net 1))
 (segment (start 150 60.89) (end 150 54.5) (width 0.2) (layer "F.Cu") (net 1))
 (segment (start 132.46 84.66) (end 127.66 84.66) (width 0.2) (layer "F.Cu") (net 1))
 (segment (start 127.5 72.5) (end 127.5 73) (width 0.2) (layer "F.Cu") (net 1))
 (segment (start 127.5 84.5) (end 127.5 96.5) (width 0.2) (layer "F.Cu") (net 1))
 (segment (start 127.5 73) (end 127.5 84.5) (width 0.2) (layer "F.Cu") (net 1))
 (segment (start 127.83 72.83) (end 127.5 72.5) (width 0.2) (layer "F.Cu") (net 1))
 (segment (start 197.5 84.5) (end 197.5 96.5) (width 0.2) (layer "F.Cu") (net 1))
 (segment (start 127.5 54.5) (end 127.5 61) (width 0.2) (layer "F.Cu") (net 1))
 (segment (start 127.5 61) (end 127.5 72.5) (width 0.2) (layer "F.Cu") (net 1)))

